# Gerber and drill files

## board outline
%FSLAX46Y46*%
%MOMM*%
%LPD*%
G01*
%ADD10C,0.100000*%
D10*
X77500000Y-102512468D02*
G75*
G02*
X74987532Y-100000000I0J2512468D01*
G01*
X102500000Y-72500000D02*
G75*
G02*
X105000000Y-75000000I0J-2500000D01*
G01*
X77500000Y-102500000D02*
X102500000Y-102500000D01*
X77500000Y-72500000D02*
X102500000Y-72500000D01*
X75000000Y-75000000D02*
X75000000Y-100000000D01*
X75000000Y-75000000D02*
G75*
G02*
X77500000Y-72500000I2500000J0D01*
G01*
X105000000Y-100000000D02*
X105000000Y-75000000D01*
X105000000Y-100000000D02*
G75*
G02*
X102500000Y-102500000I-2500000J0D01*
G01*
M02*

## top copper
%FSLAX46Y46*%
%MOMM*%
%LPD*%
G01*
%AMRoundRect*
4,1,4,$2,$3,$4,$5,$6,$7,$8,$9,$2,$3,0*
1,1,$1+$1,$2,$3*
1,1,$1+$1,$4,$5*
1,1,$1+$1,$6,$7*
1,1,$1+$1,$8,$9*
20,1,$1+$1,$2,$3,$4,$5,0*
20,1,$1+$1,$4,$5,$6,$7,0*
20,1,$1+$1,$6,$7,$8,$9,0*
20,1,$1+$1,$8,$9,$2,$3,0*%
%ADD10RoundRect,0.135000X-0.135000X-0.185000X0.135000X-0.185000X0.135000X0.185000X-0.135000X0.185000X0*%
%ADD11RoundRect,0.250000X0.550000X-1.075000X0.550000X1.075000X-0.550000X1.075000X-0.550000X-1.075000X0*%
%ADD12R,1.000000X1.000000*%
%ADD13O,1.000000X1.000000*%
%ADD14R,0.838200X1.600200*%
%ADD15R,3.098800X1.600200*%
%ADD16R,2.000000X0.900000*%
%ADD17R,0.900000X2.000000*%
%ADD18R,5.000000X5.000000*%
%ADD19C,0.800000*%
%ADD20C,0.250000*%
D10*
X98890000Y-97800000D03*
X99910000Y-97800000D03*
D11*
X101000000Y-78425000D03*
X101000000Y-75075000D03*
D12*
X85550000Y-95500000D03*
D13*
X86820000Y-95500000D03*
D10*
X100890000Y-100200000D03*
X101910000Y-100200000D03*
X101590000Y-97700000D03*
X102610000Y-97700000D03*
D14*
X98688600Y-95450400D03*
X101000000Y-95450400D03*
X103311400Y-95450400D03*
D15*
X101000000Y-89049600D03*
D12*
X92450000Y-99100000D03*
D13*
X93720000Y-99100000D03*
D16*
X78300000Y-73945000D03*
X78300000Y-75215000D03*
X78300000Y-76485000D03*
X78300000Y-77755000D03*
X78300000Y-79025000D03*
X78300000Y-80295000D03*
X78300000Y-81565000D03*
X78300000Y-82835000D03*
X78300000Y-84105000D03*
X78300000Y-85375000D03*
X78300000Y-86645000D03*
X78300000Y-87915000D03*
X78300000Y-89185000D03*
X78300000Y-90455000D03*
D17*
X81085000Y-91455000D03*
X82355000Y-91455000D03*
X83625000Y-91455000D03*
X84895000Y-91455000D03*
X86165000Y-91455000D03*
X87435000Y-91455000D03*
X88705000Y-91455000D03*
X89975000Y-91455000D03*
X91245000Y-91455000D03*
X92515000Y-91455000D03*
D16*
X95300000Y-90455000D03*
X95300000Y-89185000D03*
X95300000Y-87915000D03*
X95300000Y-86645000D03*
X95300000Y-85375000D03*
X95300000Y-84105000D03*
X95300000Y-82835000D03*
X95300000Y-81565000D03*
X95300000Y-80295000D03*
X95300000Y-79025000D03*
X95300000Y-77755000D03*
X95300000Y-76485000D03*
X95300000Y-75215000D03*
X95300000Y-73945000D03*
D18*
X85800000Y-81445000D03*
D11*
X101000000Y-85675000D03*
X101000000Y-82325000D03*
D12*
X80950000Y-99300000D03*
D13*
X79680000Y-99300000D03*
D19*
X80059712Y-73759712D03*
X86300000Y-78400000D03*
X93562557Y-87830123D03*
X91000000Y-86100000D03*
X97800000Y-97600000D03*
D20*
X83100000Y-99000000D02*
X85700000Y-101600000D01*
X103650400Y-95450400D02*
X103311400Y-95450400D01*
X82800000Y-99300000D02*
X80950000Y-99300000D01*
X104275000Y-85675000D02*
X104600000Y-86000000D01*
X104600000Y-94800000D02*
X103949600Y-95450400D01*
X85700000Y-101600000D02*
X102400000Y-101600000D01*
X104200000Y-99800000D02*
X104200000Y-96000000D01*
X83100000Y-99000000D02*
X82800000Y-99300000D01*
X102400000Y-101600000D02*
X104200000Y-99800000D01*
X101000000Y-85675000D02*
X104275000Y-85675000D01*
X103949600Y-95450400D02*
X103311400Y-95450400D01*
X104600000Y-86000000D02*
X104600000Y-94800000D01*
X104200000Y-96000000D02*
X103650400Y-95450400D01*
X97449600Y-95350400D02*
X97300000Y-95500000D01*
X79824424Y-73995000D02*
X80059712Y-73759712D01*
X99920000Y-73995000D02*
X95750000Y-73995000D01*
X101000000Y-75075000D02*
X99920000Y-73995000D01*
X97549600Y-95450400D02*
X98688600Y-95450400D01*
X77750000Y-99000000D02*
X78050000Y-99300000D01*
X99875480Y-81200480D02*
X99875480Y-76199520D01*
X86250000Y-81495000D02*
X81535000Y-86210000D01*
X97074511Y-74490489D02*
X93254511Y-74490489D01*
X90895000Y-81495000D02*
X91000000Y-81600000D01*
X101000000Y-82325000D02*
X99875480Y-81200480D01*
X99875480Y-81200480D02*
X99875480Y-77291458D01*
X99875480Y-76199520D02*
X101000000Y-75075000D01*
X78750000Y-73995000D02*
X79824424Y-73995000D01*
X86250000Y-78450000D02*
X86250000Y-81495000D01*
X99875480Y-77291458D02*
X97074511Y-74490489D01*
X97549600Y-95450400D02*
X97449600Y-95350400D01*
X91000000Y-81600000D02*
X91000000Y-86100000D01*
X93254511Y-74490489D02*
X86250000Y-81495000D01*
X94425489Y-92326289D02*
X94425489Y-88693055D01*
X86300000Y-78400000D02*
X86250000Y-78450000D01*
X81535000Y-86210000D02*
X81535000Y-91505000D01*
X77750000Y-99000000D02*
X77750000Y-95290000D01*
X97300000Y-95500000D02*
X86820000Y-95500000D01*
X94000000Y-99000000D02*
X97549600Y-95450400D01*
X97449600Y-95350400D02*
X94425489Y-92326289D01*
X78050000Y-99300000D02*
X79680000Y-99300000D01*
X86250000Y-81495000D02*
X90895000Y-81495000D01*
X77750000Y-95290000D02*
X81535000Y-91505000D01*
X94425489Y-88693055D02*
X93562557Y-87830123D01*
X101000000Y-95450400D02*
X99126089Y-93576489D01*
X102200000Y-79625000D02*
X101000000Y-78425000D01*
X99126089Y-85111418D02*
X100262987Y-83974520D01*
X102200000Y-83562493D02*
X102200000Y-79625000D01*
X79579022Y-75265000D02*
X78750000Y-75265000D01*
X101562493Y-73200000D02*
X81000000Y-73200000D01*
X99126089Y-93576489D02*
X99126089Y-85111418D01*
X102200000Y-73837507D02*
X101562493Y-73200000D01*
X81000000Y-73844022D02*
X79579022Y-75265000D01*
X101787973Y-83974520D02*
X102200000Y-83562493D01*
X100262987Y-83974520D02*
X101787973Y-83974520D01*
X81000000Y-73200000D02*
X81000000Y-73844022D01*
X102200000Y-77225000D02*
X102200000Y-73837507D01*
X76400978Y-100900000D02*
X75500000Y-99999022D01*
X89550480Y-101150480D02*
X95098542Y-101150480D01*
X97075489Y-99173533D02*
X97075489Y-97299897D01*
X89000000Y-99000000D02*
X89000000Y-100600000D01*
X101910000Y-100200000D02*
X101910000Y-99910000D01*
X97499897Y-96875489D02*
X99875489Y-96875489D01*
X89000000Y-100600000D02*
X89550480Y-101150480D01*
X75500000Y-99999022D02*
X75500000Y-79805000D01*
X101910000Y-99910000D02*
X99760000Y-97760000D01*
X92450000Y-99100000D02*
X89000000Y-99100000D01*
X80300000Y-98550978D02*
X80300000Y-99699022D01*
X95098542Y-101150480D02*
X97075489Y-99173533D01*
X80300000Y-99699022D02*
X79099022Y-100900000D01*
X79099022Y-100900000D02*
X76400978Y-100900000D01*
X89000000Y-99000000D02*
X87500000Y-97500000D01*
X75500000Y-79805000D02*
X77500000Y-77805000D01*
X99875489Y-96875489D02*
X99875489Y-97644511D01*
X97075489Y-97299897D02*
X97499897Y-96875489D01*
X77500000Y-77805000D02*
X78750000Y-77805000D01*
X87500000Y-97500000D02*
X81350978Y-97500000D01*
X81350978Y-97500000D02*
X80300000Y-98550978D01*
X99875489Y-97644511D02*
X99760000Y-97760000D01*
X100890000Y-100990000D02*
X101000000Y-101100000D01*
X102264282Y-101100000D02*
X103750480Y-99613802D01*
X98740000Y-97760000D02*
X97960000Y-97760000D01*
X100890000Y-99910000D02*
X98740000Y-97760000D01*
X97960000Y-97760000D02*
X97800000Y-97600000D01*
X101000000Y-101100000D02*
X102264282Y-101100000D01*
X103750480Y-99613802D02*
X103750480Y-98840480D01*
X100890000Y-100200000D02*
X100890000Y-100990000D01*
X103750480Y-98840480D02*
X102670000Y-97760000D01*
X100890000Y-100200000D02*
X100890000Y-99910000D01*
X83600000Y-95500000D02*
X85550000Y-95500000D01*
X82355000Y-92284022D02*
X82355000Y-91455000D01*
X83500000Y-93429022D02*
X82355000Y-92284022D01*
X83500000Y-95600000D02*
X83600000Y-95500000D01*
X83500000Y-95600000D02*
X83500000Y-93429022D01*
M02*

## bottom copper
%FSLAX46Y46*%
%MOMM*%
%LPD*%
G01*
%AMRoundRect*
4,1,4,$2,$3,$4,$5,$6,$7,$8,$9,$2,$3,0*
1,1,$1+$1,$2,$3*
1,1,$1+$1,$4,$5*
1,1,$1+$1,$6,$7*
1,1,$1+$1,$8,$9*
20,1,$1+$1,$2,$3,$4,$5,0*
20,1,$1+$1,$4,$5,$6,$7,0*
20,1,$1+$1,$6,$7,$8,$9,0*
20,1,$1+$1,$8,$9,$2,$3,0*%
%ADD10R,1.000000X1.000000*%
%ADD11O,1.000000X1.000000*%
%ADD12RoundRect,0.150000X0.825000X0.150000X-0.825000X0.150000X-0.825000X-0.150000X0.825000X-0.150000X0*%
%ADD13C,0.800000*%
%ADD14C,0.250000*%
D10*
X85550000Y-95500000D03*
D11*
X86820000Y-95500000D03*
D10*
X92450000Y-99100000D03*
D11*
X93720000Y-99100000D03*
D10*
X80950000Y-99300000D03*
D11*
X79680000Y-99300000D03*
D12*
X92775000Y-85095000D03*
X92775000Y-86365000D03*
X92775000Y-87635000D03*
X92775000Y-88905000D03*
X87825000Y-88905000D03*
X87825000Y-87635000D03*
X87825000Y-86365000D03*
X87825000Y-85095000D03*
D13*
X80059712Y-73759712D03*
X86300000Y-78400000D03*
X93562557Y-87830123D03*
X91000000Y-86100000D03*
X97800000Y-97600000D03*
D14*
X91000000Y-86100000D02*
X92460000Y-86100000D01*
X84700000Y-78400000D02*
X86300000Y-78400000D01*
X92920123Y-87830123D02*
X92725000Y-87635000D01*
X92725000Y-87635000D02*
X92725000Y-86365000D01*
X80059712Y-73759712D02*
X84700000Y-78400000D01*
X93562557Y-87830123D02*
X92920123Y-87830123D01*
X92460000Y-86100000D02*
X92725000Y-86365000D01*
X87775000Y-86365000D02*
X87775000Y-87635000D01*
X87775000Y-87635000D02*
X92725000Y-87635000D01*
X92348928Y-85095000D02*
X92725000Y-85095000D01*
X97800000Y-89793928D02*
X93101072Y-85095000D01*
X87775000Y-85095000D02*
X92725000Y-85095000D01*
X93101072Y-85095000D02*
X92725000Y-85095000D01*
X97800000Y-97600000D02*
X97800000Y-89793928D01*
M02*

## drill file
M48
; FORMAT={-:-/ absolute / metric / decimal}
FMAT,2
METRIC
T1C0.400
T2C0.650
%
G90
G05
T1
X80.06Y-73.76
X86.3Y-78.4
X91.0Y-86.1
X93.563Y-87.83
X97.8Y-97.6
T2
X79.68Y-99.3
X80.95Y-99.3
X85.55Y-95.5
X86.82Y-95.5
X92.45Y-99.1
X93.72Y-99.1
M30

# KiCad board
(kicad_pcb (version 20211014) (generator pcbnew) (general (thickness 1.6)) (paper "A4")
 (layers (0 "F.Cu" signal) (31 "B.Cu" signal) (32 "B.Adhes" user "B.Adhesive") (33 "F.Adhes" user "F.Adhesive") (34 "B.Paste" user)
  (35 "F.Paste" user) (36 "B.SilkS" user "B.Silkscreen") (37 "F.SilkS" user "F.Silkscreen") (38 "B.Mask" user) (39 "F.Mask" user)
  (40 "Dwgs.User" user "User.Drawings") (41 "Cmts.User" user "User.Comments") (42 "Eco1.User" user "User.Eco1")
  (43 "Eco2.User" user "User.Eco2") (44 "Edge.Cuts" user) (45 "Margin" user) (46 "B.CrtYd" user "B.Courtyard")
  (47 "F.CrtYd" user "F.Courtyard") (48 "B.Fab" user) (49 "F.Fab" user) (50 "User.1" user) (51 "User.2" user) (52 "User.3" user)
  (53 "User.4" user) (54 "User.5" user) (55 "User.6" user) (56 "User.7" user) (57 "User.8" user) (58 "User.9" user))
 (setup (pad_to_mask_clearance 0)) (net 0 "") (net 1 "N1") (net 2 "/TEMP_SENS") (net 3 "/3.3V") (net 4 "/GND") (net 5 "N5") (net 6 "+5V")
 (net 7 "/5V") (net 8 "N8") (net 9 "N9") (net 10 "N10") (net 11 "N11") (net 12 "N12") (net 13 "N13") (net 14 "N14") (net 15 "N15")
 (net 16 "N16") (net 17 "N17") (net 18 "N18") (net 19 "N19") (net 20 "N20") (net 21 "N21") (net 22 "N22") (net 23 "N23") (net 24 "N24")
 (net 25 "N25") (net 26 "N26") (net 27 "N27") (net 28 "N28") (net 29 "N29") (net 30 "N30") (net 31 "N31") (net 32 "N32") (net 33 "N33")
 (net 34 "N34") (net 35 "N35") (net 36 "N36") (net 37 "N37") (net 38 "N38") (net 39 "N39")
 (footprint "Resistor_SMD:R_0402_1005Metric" (layer "F.Cu") (at 99.4 97.8)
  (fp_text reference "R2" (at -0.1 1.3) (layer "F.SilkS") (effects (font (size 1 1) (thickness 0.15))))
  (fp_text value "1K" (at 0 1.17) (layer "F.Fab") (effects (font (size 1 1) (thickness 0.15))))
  (pad "1" smd roundrect (at -0.51 0) (size 0.54 0.64) (layers "F.Cu" "F.Paste" "F.Mask") (roundrect_rratio 0.25) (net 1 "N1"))
  (pad "2" smd roundrect (at 0.51 0) (size 0.54 0.64) (layers "F.Cu" "F.Paste" "F.Mask") (roundrect_rratio 0.25) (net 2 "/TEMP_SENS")))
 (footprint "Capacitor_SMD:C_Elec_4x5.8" (layer "F.Cu") (at 101 76.75 90)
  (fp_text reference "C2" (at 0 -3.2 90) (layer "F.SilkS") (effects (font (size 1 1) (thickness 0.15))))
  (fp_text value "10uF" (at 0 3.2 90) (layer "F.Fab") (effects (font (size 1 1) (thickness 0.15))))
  (pad "1" smd roundrect (at -1.675 0 90) (size 2.65 1.6) (layers "F.Cu" "F.Paste" "F.Mask") (roundrect_rratio 0.15625) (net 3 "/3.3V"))
  (pad "2" smd roundrect (at 1.675 0 90) (size 2.65 1.6) (layers "F.Cu" "F.Paste" "F.Mask") (roundrect_rratio 0.15625) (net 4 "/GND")))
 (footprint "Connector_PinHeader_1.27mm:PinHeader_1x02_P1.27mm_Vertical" (layer "F.Cu") (at 85.55 95.5 90)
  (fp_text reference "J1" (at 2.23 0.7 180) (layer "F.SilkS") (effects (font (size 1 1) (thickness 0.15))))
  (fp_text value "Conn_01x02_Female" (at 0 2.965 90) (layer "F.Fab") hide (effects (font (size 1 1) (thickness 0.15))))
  (pad "1" thru_hole rect (at 0 0 90) (size 1 1) (drill 0.65) (layers *.Cu *.Mask) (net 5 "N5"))
  (pad "2" thru_hole oval (at 0 1.27 90) (size 1 1) (drill 0.65) (layers *.Cu *.Mask) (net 4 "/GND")))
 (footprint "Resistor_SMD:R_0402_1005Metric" (layer "F.Cu") (at 101.4 100.2)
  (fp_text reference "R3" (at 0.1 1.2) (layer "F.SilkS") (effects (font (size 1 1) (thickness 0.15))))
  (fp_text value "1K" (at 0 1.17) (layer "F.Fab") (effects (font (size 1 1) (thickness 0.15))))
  (pad "1" smd roundrect (at -0.51 0) (size 0.54 0.64) (layers "F.Cu" "F.Paste" "F.Mask") (roundrect_rratio 0.25) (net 1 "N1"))
  (pad "2" smd roundrect (at 0.51 0) (size 0.54 0.64) (layers "F.Cu" "F.Paste" "F.Mask") (roundrect_rratio 0.25) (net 2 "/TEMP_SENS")))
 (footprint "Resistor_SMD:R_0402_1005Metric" (layer "F.Cu") (at 102.1 97.7)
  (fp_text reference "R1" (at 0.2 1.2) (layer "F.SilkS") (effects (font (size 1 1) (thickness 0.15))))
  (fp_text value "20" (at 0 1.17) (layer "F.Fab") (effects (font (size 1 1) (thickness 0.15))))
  (pad "1" smd roundrect (at -0.51 0) (size 0.54 0.64) (layers "F.Cu" "F.Paste" "F.Mask") (roundrect_rratio 0.25) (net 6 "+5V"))
  (pad "2" smd roundrect (at 0.51 0) (size 0.54 0.64) (layers "F.Cu" "F.Paste" "F.Mask") (roundrect_rratio 0.25) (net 1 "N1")))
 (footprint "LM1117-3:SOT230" (layer "F.Cu") (at 101 92.25 90)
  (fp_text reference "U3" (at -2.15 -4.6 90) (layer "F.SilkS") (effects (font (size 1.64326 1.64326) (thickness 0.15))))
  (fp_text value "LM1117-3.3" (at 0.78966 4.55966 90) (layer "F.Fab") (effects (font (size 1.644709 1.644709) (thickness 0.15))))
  (pad "1" smd rect locked (at -3.2004 -2.3114 90) (size 1.6002 0.8382) (layers "F.Cu" "F.Paste" "F.Mask") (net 4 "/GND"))
  (pad "2" smd rect locked (at -3.2004 0 90) (size 1.6002 0.8382) (layers "F.Cu" "F.Paste" "F.Mask") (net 3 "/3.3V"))
  (pad "3" smd rect locked (at -3.2004 2.3114 90) (size 1.6002 0.8382) (layers "F.Cu" "F.Paste" "F.Mask") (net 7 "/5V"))
  (pad "4" smd rect locked (at 3.2004 0 90) (size 1.6002 3.0988) (layers "F.Cu" "F.Paste" "F.Mask")))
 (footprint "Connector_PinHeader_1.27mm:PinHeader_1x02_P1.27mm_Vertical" (layer "F.Cu") (at 92.45 99.1 90)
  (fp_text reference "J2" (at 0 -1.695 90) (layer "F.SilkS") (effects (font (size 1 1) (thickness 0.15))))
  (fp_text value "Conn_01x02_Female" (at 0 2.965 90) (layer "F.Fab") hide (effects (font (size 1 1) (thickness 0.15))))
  (pad "1" thru_hole rect (at 0 0 90) (size 1 1) (drill 0.65) (layers *.Cu *.Mask) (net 2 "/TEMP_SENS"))
  (pad "2" thru_hole oval (at 0 1.27 90) (size 1 1) (drill 0.65) (layers *.Cu *.Mask) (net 4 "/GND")))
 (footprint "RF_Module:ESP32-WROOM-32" (layer "F.Cu") (at 86.8 82.2)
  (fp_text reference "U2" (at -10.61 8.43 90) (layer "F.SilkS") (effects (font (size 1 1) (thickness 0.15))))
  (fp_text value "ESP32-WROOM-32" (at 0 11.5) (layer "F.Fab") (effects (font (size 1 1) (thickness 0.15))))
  (pad "1" smd rect (at -8.5 -8.255) (size 2 0.9) (layers "F.Cu" "F.Paste" "F.Mask") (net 4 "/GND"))
  (pad "2" smd rect (at -8.5 -6.985) (size 2 0.9) (layers "F.Cu" "F.Paste" "F.Mask") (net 3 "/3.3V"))
  (pad "3" smd rect (at -8.5 -5.715) (size 2 0.9) (layers "F.Cu" "F.Paste" "F.Mask") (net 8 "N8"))
  (pad "4" smd rect (at -8.5 -4.445) (size 2 0.9) (layers "F.Cu" "F.Paste" "F.Mask") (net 2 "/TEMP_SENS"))
  (pad "5" smd rect (at -8.5 -3.175) (size 2 0.9) (layers "F.Cu" "F.Paste" "F.Mask") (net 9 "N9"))
  (pad "6" smd rect (at -8.5 -1.905) (size 2 0.9) (layers "F.Cu" "F.Paste" "F.Mask") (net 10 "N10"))
  (pad "7" smd rect (at -8.5 -0.635) (size 2 0.9) (layers "F.Cu" "F.Paste" "F.Mask") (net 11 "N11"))
  (pad "8" smd rect (at -8.5 0.635) (size 2 0.9) (layers "F.Cu" "F.Paste" "F.Mask") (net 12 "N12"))
  (pad "9" smd rect (at -8.5 1.905) (size 2 0.9) (layers "F.Cu" "F.Paste" "F.Mask") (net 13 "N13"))
  (pad "10" smd rect (at -8.5 3.175) (size 2 0.9) (layers "F.Cu" "F.Paste" "F.Mask") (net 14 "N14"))
  (pad "11" smd rect (at -8.5 4.445) (size 2 0.9) (layers "F.Cu" "F.Paste" "F.Mask") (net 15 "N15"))
  (pad "12" smd rect (at -8.5 5.715) (size 2 0.9) (layers "F.Cu" "F.Paste" "F.Mask") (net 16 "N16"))
  (pad "13" smd rect (at -8.5 6.985) (size 2 0.9) (layers "F.Cu" "F.Paste" "F.Mask") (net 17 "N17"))
  (pad "14" smd rect (at -8.5 8.255) (size 2 0.9) (layers "F.Cu" "F.Paste" "F.Mask") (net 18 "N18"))
  (pad "15" smd rect (at -5.715 9.255 90) (size 2 0.9) (layers "F.Cu" "F.Paste" "F.Mask") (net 4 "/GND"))
  (pad "16" smd rect (at -4.445 9.255 90) (size 2 0.9) (layers "F.Cu" "F.Paste" "F.Mask") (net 5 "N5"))
  (pad "17" smd rect (at -3.175 9.255 90) (size 2 0.9) (layers "F.Cu" "F.Paste" "F.Mask") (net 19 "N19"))
  (pad "18" smd rect (at -1.905 9.255 90) (size 2 0.9) (layers "F.Cu" "F.Paste" "F.Mask") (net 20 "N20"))
  (pad "19" smd rect (at -0.635 9.255 90) (size 2 0.9) (layers "F.Cu" "F.Paste" "F.Mask") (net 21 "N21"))
  (pad "20" smd rect (at 0.635 9.255 90) (size 2 0.9) (layers "F.Cu" "F.Paste" "F.Mask") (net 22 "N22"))
  (pad "21" smd rect (at 1.905 9.255 90) (size 2 0.9) (layers "F.Cu" "F.Paste" "F.Mask") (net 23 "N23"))
  (pad "22" smd rect (at 3.175 9.255 90) (size 2 0.9) (layers "F.Cu" "F.Paste" "F.Mask") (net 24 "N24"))
  (pad "23" smd rect (at 4.445 9.255 90) (size 2 0.9) (layers "F.Cu" "F.Paste" "F.Mask") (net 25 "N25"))
  (pad "24" smd rect (at 5.715 9.255 90) (size 2 0.9) (layers "F.Cu" "F.Paste" "F.Mask") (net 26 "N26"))
  (pad "25" smd rect (at 8.5 8.255) (size 2 0.9) (layers "F.Cu" "F.Paste" "F.Mask") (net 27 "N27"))
  (pad "26" smd rect (at 8.5 6.985) (size 2 0.9) (layers "F.Cu" "F.Paste" "F.Mask") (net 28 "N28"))
  (pad "27" smd rect (at 8.5 5.715) (size 2 0.9) (layers "F.Cu" "F.Paste" "F.Mask") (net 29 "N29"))
  (pad "28" smd rect (at 8.5 4.445) (size 2 0.9) (layers "F.Cu" "F.Paste" "F.Mask") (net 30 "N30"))
  (pad "29" smd rect (at 8.5 3.175) (size 2 0.9) (layers "F.Cu" "F.Paste" "F.Mask") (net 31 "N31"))
  (pad "30" smd rect (at 8.5 1.905) (size 2 0.9) (layers "F.Cu" "F.Paste" "F.Mask") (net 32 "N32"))
  (pad "31" smd rect (at 8.5 0.635) (size 2 0.9) (layers "F.Cu" "F.Paste" "F.Mask") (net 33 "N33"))
  (pad "32" smd rect (at 8.5 -0.635) (size 2 0.9) (layers "F.Cu" "F.Paste" "F.Mask") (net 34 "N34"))
  (pad "33" smd rect (at 8.5 -1.905) (size 2 0.9) (layers "F.Cu" "F.Paste" "F.Mask") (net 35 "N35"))
  (pad "34" smd rect (at 8.5 -3.175) (size 2 0.9) (layers "F.Cu" "F.Paste" "F.Mask") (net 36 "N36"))
  (pad "35" smd rect (at 8.5 -4.445) (size 2 0.9) (layers "F.Cu" "F.Paste" "F.Mask") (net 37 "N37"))
  (pad "36" smd rect (at 8.5 -5.715) (size 2 0.9) (layers "F.Cu" "F.Paste" "F.Mask") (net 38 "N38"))
  (pad "37" smd rect (at 8.5 -6.985) (size 2 0.9) (layers "F.Cu" "F.Paste" "F.Mask") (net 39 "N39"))
  (pad "38" smd rect (at 8.5 -8.255) (size 2 0.9) (layers "F.Cu" "F.Paste" "F.Mask") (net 4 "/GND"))
  (pad "39" smd rect (at -1 -0.755) (size 5 5) (layers "F.Cu" "F.Paste" "F.Mask") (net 4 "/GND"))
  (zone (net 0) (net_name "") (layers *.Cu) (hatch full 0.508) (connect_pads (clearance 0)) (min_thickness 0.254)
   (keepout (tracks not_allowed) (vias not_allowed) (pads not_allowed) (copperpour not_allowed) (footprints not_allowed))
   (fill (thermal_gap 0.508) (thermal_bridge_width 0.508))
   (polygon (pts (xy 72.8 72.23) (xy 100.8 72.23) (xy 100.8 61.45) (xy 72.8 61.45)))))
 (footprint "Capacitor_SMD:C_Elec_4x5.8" (layer "F.Cu") (at 101 84 90)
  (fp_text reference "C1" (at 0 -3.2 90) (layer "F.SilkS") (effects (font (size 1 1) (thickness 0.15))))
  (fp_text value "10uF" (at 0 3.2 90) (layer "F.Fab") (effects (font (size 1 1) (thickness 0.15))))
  (pad "1" smd roundrect (at -1.675 0 90) (size 2.65 1.6) (layers "F.Cu" "F.Paste" "F.Mask") (roundrect_rratio 0.15625) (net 7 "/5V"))
  (pad "2" smd roundrect (at 1.675 0 90) (size 2.65 1.6) (layers "F.Cu" "F.Paste" "F.Mask") (roundrect_rratio 0.15625) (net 4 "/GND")))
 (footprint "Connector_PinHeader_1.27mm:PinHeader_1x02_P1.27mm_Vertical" (layer "F.Cu") (at 80.95 99.3 -90)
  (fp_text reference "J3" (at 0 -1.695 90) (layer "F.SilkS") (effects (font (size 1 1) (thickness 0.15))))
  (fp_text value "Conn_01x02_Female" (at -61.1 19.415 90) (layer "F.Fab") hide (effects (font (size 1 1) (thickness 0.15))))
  (pad "1" thru_hole rect (at 0 0 270) (size 1 1) (drill 0.65) (layers *.Cu *.Mask) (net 7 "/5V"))
  (pad "2" thru_hole oval (at 0 1.27 270) (size 1 1) (drill 0.65) (layers *.Cu *.Mask) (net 4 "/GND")))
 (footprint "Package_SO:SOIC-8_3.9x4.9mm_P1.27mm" (layer "B.Cu") (at 90.3 87 180)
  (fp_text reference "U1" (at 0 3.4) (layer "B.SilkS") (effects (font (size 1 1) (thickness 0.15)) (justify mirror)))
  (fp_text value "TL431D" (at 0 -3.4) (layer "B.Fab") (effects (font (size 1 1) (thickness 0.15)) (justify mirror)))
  (pad "1" smd roundrect (at -2.475 1.905 180) (size 1.95 0.6) (layers "B.Cu" "B.Paste" "B.Mask") (roundrect_rratio 0.25) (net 1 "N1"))
  (pad "2" smd roundrect (at -2.475 0.635 180) (size 1.95 0.6) (layers "B.Cu" "B.Paste" "B.Mask") (roundrect_rratio 0.25) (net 4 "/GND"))
  (pad "3" smd roundrect (at -2.475 -0.635 180) (size 1.95 0.6) (layers "B.Cu" "B.Paste" "B.Mask") (roundrect_rratio 0.25) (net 4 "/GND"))
  (pad "4" smd roundrect (at -2.475 -1.905 180) (size 1.95 0.6) (layers "B.Cu" "B.Paste" "B.Mask") (roundrect_rratio 0.25))
  (pad "5" smd roundrect (at 2.475 -1.905 180) (size 1.95 0.6) (layers "B.Cu" "B.Paste" "B.Mask") (roundrect_rratio 0.25))
  (pad "6" smd roundrect (at 2.475 -0.635 180) (size 1.95 0.6) (layers "B.Cu" "B.Paste" "B.Mask") (roundrect_rratio 0.25) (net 4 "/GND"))
  (pad "7" smd roundrect (at 2.475 0.635 180) (size 1.95 0.6) (layers "B.Cu" "B.Paste" "B.Mask") (roundrect_rratio 0.25) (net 4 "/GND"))
  (pad "8" smd roundrect (at 2.475 1.905 180) (size 1.95 0.6) (layers "B.Cu" "B.Paste" "B.Mask") (roundrect_rratio 0.25) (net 1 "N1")))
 (gr_arc (start 77.5 102.512468) (mid 75.723417 101.776583) (end 74.987532 100) (layer "Edge.Cuts") (width 0.1))
 (gr_arc (start 102.5 72.5) (mid 104.267767 73.232233) (end 105 75) (layer "Edge.Cuts") (width 0.1))
 (gr_line (start 77.5 102.5) (end 102.5 102.5) (layer "Edge.Cuts") (width 0.1))
 (gr_line (start 77.5 72.5) (end 102.5 72.5) (layer "Edge.Cuts") (width 0.1))
 (gr_line (start 75 75) (end 75 100) (layer "Edge.Cuts") (width 0.1))
 (gr_arc (start 75 75) (mid 75.732233 73.232233) (end 77.5 72.5) (layer "Edge.Cuts") (width 0.1))
 (gr_line (start 105 100) (end 105 75) (layer "Edge.Cuts") (width 0.1))
 (gr_arc (start 105 100) (mid 104.267767 101.767767) (end 102.5 102.5) (layer "Edge.Cuts") (width 0.1))
 (segment (start 83.1 99) (end 85.7 101.6) (width 0.25) (layer "F.Cu") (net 7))
 (segment (start 103.6504 95.4504) (end 103.3114 95.4504) (width 0.25) (layer "F.Cu") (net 7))
 (segment (start 82.8 99.3) (end 80.95 99.3) (width 0.25) (layer "F.Cu") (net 7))
 (segment (start 104.275 85.675) (end 104.6 86) (width 0.25) (layer "F.Cu") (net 7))
 (segment (start 104.6 94.8) (end 103.9496 95.4504) (width 0.25) (layer "F.Cu") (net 7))
 (segment (start 85.7 101.6) (end 102.4 101.6) (width 0.25) (layer "F.Cu") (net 7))
 (segment (start 104.2 99.8) (end 104.2 96) (width 0.25) (layer "F.Cu") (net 7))
 (segment (start 83.1 99) (end 82.8 99.3) (width 0.25) (layer "F.Cu") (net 7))
 (segment (start 102.4 101.6) (end 104.2 99.8) (width 0.25) (layer "F.Cu") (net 7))
 (segment (start 101 85.675) (end 104.275 85.675) (width 0.25) (layer "F.Cu") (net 7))
 (segment (start 103.9496 95.4504) (end 103.3114 95.4504) (width 0.25) (layer "F.Cu") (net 7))
 (segment (start 104.6 86) (end 104.6 94.8) (width 0.25) (layer "F.Cu") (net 7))
 (segment (start 104.2 96) (end 103.6504 95.4504) (width 0.25) (layer "F.Cu") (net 7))
 (segment (start 97.4496 95.3504) (end 97.3 95.5) (width 0.25) (layer "F.Cu") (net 4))
 (segment (start 79.824424 73.995) (end 80.059712 73.759712) (width 0.25) (layer "F.Cu") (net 4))
 (segment (start 99.92 73.995) (end 95.75 73.995) (width 0.25) (layer "F.Cu") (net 4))
 (segment (start 101 75.075) (end 99.92 73.995) (width 0.25) (layer "F.Cu") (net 4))
 (segment (start 97.5496 95.4504) (end 98.6886 95.4504) (width 0.25) (layer "F.Cu") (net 4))
 (segment (start 77.75 99) (end 78.05 99.3) (width 0.25) (layer "F.Cu") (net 4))
 (segment (start 99.87548 81.20048) (end 99.87548 76.19952) (width 0.25) (layer "F.Cu") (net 4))
 (segment (start 86.25 81.495) (end 81.535 86.21) (width 0.25) (layer "F.Cu") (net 4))
 (segment (start 97.074511 74.490489) (end 93.254511 74.490489) (width 0.25) (layer "F.Cu") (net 4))
 (segment (start 90.895 81.495) (end 91 81.6) (width 0.25) (layer "F.Cu") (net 4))
 (segment (start 101 82.325) (end 99.87548 81.20048) (width 0.25) (layer "F.Cu") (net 4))
 (segment (start 99.87548 81.20048) (end 99.87548 77.291458) (width 0.25) (layer "F.Cu") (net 4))
 (segment (start 99.87548 76.19952) (end 101 75.075) (width 0.25) (layer "F.Cu") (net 4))
 (segment (start 78.75 73.995) (end 79.824424 73.995) (width 0.25) (layer "F.Cu") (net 4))
 (segment (start 86.25 78.45) (end 86.25 81.495) (width 0.25) (layer "F.Cu") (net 4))
 (segment (start 99.87548 77.291458) (end 97.074511 74.490489) (width 0.25) (layer "F.Cu") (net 4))
 (segment (start 97.5496 95.4504) (end 97.4496 95.3504) (width 0.25) (layer "F.Cu") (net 4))
 (segment (start 91 81.6) (end 91 86.1) (width 0.25) (layer "F.Cu") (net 4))
 (segment (start 93.254511 74.490489) (end 86.25 81.495) (width 0.25) (layer "F.Cu") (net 4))
 (segment (start 94.425489 92.326289) (end 94.425489 88.693055) (width 0.25) (layer "F.Cu") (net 4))
 (segment (start 86.3 78.4) (end 86.25 78.45) (width 0.25) (layer "F.Cu") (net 4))
 (segment (start 81.535 86.21) (end 81.535 91.505) (width 0.25) (layer "F.Cu") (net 4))
 (segment (start 77.75 99) (end 77.75 95.29) (width 0.25) (layer "F.Cu") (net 4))
 (segment (start 97.3 95.5) (end 86.82 95.5) (width 0.25) (layer "F.Cu") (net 4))
 (segment (start 94 99) (end 97.5496 95.4504) (width 0.25) (layer "F.Cu") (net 4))
 (segment (start 97.4496 95.3504) (end 94.425489 92.326289) (width 0.25) (layer "F.Cu") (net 4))
 (segment (start 78.05 99.3) (end 79.68 99.3) (width 0.25) (layer "F.Cu") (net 4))
 (segment (start 86.25 81.495) (end 90.895 81.495) (width 0.25) (layer "F.Cu") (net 4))
 (segment (start 77.75 95.29) (end 81.535 91.505) (width 0.25) (layer "F.Cu") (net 4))
 (segment (start 94.425489 88.693055) (end 93.562557 87.830123) (width 0.25) (layer "F.Cu") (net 4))
 (via (at 80.059712 73.759712) (size 0.8) (drill 0.4) (layers "F.Cu" "B.Cu") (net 4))
 (via (at 86.3 78.4) (size 0.8) (drill 0.4) (layers "F.Cu" "B.Cu") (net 4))
 (via (at 93.562557 87.830123) (size 0.8) (drill 0.4) (layers "F.Cu" "B.Cu") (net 4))
 (via (at 91 86.1) (size 0.8) (drill 0.4) (layers "F.Cu" "B.Cu") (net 4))
 (segment (start 91 86.1) (end 92.46 86.1) (width 0.25) (layer "B.Cu") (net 4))
 (segment (start 84.7 78.4) (end 86.3 78.4) (width 0.25) (layer "B.Cu") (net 4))
 (segment (start 92.920123 87.830123) (end 92.725 87.635) (width 0.25) (layer "B.Cu") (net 4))
 (segment (start 92.725 87.635) (end 92.725 86.365) (width 0.25) (layer "B.Cu") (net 4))
 (segment (start 80.059712 73.759712) (end 84.7 78.4) (width 0.25) (layer "B.Cu") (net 4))
 (segment (start 93.562557 87.830123) (end 92.920123 87.830123) (width 0.25) (layer "B.Cu") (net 4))
 (segment (start 92.46 86.1) (end 92.725 86.365) (width 0.25) (layer "B.Cu") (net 4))
 (segment (start 87.775 86.365) (end 87.775 87.635) (width 0.25) (layer "B.Cu") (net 4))
 (segment (start 87.775 87.635) (end 92.725 87.635) (width 0.25) (layer "B.Cu") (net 4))
 (segment (start 101 95.4504) (end 99.126089 93.576489) (width 0.25) (layer "F.Cu") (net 3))
 (segment (start 102.2 79.625) (end 101 78.425) (width 0.25) (layer "F.Cu") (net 3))
 (segment (start 99.126089 85.111418) (end 100.262987 83.97452) (width 0.25) (layer "F.Cu") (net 3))
 (segment (start 102.2 83.562493) (end 102.2 79.625) (width 0.25) (layer "F.Cu") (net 3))
 (segment (start 79.579022 75.265) (end 78.75 75.265) (width 0.25) (layer "F.Cu") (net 3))
 (segment (start 101.562493 73.2) (end 81 73.2) (width 0.25) (layer "F.Cu") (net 3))
 (segment (start 99.126089 93.576489) (end 99.126089 85.111418) (width 0.25) (layer "F.Cu") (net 3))
 (segment (start 102.2 73.837507) (end 101.562493 73.2) (width 0.25) (layer "F.Cu") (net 3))
 (segment (start 81 73.844022) (end 79.579022 75.265) (width 0.25) (layer "F.Cu") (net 3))
 (segment (start 101.787973 83.97452) (end 102.2 83.562493) (width 0.25) (layer "F.Cu") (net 3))
 (segment (start 100.262987 83.97452) (end 101.787973 83.97452) (width 0.25) (layer "F.Cu") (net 3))
 (segment (start 81 73.2) (end 81 73.844022) (width 0.25) (layer "F.Cu") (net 3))
 (segment (start 102.2 77.225) (end 102.2 73.837507) (width 0.25) (layer "F.Cu") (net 3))
 (segment (start 76.400978 100.9) (end 75.5 99.999022) (width 0.25) (layer "F.Cu") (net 2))
 (segment (start 89.55048 101.15048) (end 95.098542 101.15048) (width 0.25) (layer "F.Cu") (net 2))
 (segment (start 97.075489 99.173533) (end 97.075489 97.299897) (width 0.25) (layer "F.Cu") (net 2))
 (segment (start 89 99) (end 89 100.6) (width 0.25) (layer "F.Cu") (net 2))
 (segment (start 101.91 100.2) (end 101.91 99.91) (width 0.25) (layer "F.Cu") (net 2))
 (segment (start 97.499897 96.875489) (end 99.875489 96.875489) (width 0.25) (layer "F.Cu") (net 2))
 (segment (start 89 100.6) (end 89.55048 101.15048) (width 0.25) (layer "F.Cu") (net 2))
 (segment (start 75.5 99.999022) (end 75.5 79.805) (width 0.25) (layer "F.Cu") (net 2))
 (segment (start 101.91 99.91) (end 99.76 97.76) (width 0.25) (layer "F.Cu") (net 2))
 (segment (start 92.45 99.1) (end 89 99.1) (width 0.25) (layer "F.Cu") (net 2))
 (segment (start 80.3 98.550978) (end 80.3 99.699022) (width 0.25) (layer "F.Cu") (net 2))
 (segment (start 95.098542 101.15048) (end 97.075489 99.173533) (width 0.25) (layer "F.Cu") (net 2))
 (segment (start 80.3 99.699022) (end 79.099022 100.9) (width 0.25) (layer "F.Cu") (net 2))
 (segment (start 79.099022 100.9) (end 76.400978 100.9) (width 0.25) (layer "F.Cu") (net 2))
 (segment (start 89 99) (end 87.5 97.5) (width 0.25) (layer "F.Cu") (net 2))
 (segment (start 75.5 79.805) (end 77.5 77.805) (width 0.25) (layer "F.Cu") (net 2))
 (segment (start 99.875489 96.875489) (end 99.875489 97.644511) (width 0.25) (layer "F.Cu") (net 2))
 (segment (start 97.075489 97.299897) (end 97.499897 96.875489) (width 0.25) (layer "F.Cu") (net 2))
 (segment (start 77.5 77.805) (end 78.75 77.805) (width 0.25) (layer "F.Cu") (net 2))
 (segment (start 87.5 97.5) (end 81.350978 97.5) (width 0.25) (layer "F.Cu") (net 2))
 (segment (start 81.350978 97.5) (end 80.3 98.550978) (width 0.25) (layer "F.Cu") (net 2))
 (segment (start 99.875489 97.644511) (end 99.76 97.76) (width 0.25) (layer "F.Cu") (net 2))
 (segment (start 100.89 100.99) (end 101 101.1) (width 0.25) (layer "F.Cu") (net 1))
 (segment (start 102.264282 101.1) (end 103.75048 99.613802) (width 0.25) (layer "F.Cu") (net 1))
 (segment (start 98.74 97.76) (end 97.96 97.76) (width 0.25) (layer "F.Cu") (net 1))
 (segment (start 100.89 99.91) (end 98.74 97.76) (width 0.25) (layer "F.Cu") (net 1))
 (segment (start 97.96 97.76) (end 97.8 97.6) (width 0.25) (layer "F.Cu") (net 1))
 (segment (start 101 101.1) (end 102.264282 101.1) (width 0.25) (layer "F.Cu") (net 1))
 (segment (start 103.75048 99.613802) (end 103.75048 98.84048) (width 0.25) (layer "F.Cu") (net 1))
 (segment (start 100.89 100.2) (end 100.89 100.99) (width 0.25) (layer "F.Cu") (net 1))
 (segment (start 103.75048 98.84048) (end 102.67 97.76) (width 0.25) (layer "F.Cu") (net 1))
 (segment (start 100.89 100.2) (end 100.89 99.91) (width 0.25) (layer "F.Cu") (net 1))
 (via (at 97.8 97.6) (size 0.8) (drill 0.4) (layers "F.Cu" "B.Cu") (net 1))
 (segment (start 92.348928 85.095) (end 92.725 85.095) (width 0.25) (layer "B.Cu") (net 1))
 (segment (start 97.8 89.793928) (end 93.101072 85.095) (width 0.25) (layer "B.Cu") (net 1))
 (segment (start 87.775 85.095) (end 92.725 85.095) (width 0.25) (layer "B.Cu") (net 1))
 (segment (start 93.101072 85.095) (end 92.725 85.095) (width 0.25) (layer "B.Cu") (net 1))
 (segment (start 97.8 97.6) (end 97.8 89.793928) (width 0.25) (layer "B.Cu") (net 1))
 (segment (start 83.6 95.5) (end 85.55 95.5) (width 0.25) (layer "F.Cu") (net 5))
 (segment (start 82.355 92.284022) (end 82.355 91.455) (width 0.25) (layer "F.Cu") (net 5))
 (segment (start 83.5 93.429022) (end 82.355 92.284022) (width 0.25) (layer "F.Cu") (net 5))
 (segment (start 83.5 95.6) (end 83.6 95.5) (width 0.25) (layer "F.Cu") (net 5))
 (segment (start 83.5 95.6) (end 83.5 93.429022) (width 0.25) (layer "F.Cu") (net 5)))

